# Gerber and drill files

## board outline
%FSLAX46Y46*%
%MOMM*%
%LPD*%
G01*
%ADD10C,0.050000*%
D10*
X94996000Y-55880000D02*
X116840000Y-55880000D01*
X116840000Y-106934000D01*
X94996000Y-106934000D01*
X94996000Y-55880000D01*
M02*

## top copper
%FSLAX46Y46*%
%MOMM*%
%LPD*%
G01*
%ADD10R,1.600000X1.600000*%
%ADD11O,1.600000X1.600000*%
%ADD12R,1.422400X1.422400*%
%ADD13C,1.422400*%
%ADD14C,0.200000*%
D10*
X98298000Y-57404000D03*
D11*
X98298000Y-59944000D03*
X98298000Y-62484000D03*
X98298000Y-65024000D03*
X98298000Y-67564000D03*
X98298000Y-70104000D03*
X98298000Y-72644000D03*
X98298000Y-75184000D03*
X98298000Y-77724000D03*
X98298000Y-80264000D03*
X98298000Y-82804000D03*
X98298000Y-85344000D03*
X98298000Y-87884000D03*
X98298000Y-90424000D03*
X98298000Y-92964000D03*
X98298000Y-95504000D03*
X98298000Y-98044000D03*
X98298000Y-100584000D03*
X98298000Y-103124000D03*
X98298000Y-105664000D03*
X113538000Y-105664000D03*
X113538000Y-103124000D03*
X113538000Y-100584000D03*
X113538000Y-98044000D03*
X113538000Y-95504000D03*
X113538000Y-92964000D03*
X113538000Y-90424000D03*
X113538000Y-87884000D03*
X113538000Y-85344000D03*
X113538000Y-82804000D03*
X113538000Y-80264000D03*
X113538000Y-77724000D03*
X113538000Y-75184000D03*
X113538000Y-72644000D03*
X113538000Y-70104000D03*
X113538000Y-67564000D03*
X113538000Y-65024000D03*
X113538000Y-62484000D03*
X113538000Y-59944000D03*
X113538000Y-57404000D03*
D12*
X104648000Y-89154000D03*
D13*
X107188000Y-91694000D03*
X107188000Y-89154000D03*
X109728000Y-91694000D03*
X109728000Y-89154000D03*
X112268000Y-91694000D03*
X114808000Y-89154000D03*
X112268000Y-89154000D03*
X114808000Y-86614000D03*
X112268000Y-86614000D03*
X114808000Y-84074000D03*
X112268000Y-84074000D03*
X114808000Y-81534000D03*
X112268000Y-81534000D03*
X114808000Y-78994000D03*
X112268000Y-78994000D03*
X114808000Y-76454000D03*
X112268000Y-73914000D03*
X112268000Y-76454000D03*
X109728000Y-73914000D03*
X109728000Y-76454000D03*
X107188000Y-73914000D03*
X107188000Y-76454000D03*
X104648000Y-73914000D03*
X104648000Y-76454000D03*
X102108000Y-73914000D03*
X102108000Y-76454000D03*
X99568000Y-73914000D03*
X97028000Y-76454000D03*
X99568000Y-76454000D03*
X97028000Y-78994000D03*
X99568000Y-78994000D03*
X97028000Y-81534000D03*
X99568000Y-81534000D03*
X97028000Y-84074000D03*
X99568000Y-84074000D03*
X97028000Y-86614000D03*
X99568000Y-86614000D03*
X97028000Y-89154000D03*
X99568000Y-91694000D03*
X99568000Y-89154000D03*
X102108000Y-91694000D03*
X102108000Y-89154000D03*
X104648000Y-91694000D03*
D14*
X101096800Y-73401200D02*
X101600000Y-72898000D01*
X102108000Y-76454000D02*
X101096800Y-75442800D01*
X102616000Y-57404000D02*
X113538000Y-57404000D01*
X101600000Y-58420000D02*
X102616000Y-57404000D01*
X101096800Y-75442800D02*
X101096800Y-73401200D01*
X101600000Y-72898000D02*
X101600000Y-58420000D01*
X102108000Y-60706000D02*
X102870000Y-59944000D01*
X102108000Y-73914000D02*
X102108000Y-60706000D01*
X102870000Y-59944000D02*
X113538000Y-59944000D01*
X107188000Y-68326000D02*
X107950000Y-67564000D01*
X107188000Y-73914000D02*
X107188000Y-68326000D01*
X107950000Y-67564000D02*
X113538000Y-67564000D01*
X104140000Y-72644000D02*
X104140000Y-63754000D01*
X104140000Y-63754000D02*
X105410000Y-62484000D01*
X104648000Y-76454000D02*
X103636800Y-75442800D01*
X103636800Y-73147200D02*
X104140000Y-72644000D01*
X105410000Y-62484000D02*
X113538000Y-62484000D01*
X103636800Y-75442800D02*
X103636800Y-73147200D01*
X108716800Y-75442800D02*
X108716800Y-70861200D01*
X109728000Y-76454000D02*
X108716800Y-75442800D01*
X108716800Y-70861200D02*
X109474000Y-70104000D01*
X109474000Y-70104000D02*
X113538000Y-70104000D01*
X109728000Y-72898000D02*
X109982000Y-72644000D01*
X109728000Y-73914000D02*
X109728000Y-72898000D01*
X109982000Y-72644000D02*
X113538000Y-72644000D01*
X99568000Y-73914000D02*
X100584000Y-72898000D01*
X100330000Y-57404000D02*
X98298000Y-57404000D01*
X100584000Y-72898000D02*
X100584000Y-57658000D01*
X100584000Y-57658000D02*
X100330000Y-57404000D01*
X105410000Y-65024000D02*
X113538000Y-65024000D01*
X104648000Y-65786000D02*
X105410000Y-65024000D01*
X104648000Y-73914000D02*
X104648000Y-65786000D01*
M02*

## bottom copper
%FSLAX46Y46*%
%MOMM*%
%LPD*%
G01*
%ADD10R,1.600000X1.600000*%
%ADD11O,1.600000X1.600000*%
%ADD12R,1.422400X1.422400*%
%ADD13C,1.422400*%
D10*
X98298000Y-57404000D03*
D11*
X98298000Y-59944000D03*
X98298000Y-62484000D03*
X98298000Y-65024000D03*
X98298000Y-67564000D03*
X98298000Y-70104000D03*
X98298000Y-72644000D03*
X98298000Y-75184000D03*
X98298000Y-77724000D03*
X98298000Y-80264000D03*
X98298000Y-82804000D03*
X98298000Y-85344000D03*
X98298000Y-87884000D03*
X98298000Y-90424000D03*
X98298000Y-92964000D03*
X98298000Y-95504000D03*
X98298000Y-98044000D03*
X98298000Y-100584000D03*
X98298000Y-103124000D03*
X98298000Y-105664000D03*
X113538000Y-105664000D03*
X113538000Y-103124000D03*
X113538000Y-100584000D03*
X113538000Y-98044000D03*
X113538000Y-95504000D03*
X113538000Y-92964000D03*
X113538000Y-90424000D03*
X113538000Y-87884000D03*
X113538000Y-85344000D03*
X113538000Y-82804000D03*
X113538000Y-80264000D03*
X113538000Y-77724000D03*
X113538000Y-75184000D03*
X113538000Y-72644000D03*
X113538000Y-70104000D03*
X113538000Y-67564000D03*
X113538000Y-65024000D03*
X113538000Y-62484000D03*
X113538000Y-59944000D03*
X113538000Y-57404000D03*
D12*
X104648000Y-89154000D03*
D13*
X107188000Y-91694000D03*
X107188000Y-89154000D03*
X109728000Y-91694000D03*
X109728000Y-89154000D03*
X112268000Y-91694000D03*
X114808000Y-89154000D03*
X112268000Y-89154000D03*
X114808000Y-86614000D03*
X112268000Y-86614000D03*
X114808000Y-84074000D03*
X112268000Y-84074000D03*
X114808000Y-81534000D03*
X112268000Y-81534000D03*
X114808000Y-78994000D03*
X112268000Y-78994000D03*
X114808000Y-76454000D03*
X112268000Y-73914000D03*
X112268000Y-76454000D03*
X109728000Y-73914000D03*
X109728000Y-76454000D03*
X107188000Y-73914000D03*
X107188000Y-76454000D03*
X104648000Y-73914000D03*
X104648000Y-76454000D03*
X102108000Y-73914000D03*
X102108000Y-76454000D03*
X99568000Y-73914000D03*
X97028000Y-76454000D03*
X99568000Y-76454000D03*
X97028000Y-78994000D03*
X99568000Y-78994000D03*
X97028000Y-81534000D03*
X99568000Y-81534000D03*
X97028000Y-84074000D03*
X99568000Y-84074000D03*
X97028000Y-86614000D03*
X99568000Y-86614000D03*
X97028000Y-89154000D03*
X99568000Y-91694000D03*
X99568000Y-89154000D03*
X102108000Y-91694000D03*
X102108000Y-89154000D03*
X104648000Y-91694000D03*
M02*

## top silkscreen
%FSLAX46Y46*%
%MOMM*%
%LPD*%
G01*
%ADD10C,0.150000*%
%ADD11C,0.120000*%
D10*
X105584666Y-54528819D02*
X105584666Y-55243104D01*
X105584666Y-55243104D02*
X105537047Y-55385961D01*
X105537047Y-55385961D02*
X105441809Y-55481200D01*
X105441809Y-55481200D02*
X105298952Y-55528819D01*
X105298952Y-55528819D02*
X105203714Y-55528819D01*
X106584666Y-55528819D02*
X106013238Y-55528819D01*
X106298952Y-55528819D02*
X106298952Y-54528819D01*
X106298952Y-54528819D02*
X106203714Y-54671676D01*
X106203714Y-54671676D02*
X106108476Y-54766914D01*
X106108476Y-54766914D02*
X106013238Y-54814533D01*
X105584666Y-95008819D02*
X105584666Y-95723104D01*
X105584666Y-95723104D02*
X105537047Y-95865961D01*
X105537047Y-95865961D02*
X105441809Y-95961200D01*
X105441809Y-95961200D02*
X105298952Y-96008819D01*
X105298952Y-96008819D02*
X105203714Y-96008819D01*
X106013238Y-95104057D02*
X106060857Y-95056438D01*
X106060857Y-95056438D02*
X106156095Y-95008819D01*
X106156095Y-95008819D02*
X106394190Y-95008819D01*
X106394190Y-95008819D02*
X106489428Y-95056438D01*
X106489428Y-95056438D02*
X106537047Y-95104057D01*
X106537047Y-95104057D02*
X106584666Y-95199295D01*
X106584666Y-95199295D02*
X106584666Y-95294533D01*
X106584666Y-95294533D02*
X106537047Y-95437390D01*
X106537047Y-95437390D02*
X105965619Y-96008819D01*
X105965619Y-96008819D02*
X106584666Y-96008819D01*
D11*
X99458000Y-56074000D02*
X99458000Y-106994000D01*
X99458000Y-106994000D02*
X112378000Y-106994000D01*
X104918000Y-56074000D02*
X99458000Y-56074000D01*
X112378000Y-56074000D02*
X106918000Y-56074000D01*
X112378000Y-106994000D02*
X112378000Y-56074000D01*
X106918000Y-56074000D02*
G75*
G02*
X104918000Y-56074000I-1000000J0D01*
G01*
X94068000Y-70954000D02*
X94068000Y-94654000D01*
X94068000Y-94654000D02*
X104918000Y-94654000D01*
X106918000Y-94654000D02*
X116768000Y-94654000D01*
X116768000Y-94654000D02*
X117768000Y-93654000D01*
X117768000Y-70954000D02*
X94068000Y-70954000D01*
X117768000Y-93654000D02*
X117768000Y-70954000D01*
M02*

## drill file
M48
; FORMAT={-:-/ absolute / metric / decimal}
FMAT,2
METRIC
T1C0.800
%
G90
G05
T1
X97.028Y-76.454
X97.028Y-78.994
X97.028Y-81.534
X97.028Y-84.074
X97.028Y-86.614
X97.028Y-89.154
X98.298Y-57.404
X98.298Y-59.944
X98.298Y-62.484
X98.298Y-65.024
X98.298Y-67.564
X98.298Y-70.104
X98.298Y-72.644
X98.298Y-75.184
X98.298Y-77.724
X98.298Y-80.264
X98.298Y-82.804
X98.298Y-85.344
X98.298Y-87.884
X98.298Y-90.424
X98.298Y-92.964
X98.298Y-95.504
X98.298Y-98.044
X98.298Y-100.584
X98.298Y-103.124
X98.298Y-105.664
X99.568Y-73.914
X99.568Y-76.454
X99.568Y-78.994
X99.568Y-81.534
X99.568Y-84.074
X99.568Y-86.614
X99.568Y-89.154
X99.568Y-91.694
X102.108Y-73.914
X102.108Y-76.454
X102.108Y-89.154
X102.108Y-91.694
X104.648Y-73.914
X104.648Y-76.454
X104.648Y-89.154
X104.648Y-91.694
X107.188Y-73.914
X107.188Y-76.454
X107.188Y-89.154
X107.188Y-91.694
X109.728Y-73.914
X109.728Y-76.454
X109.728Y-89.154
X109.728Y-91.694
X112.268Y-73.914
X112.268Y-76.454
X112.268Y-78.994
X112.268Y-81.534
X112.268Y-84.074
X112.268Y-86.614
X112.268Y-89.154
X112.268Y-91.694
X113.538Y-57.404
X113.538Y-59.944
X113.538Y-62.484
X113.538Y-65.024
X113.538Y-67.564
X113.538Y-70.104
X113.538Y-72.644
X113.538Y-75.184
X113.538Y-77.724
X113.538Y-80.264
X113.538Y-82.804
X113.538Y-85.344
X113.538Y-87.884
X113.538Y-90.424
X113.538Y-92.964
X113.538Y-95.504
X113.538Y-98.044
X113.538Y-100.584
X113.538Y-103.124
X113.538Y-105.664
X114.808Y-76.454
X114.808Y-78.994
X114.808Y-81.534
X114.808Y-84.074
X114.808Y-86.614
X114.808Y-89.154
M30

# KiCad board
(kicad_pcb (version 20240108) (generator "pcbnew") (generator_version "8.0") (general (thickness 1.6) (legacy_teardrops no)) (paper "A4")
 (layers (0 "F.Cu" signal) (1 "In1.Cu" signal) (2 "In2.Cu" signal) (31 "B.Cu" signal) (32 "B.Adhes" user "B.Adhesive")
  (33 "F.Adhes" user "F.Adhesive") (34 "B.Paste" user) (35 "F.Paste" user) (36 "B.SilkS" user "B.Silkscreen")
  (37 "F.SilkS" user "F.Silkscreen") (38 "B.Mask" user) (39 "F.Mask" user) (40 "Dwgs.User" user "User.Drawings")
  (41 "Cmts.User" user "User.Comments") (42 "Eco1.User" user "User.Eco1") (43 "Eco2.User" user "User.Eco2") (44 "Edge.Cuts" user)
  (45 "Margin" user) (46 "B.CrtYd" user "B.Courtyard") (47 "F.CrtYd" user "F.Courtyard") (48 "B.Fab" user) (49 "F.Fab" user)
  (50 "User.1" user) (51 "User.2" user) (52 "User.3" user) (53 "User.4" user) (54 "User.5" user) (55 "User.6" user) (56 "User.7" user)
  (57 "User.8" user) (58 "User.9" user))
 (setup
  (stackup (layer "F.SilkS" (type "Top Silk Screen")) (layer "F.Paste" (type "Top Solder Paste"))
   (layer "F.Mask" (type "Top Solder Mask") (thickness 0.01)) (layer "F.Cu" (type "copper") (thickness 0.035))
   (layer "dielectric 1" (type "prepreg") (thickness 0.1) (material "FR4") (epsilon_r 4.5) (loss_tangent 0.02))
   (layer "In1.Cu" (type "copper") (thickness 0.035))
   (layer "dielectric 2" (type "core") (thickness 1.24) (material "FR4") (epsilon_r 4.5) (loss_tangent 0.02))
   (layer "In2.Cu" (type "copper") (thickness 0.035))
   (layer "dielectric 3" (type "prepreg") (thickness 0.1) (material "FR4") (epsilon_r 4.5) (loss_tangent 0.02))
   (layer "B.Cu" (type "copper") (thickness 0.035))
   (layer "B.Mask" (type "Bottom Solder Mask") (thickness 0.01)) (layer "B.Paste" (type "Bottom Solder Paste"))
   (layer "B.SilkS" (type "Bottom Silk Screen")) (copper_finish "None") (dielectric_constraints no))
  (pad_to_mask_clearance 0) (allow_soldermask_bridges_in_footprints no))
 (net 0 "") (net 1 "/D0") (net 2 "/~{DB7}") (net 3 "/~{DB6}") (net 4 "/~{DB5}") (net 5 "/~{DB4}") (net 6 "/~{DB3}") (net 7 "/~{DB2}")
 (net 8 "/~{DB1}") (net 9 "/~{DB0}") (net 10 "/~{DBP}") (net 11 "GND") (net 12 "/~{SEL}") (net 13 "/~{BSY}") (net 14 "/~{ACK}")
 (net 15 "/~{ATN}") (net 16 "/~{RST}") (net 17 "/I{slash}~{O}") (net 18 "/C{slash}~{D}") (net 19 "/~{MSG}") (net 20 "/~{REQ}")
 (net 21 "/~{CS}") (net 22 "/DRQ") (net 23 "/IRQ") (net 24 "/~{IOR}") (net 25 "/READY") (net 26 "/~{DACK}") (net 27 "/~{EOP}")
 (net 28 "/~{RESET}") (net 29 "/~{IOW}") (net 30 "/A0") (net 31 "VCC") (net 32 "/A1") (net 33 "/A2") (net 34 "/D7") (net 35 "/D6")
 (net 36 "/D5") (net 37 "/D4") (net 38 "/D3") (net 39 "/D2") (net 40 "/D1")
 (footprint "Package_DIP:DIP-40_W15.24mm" (layer "F.Cu") (at 98.298 57.404)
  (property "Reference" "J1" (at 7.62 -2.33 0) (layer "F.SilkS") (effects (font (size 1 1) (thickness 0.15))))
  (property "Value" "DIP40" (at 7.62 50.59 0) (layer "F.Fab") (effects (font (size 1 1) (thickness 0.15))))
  (fp_line (start 1.16 -1.33) (end 1.16 49.59) (stroke (width 0.12) (type solid)) (layer "F.SilkS"))
  (fp_line (start 1.16 49.59) (end 14.08 49.59) (stroke (width 0.12) (type solid)) (layer "F.SilkS"))
  (fp_line (start 6.62 -1.33) (end 1.16 -1.33) (stroke (width 0.12) (type solid)) (layer "F.SilkS"))
  (fp_line (start 14.08 -1.33) (end 8.62 -1.33) (stroke (width 0.12) (type solid)) (layer "F.SilkS"))
  (fp_line (start 14.08 49.59) (end 14.08 -1.33) (stroke (width 0.12) (type solid)) (layer "F.SilkS"))
  (fp_arc (start 8.62 -1.33) (mid 7.62 -0.33) (end 6.62 -1.33) (stroke (width 0.12) (type solid)) (layer "F.SilkS"))
  (pad "1" thru_hole rect (at 0 0) (size 1.6 1.6) (drill 0.8) (layers "*.Cu" "*.Mask") (remove_unused_layers no) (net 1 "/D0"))
  (pad "2" thru_hole oval (at 0 2.54) (size 1.6 1.6) (drill 0.8) (layers "*.Cu" "*.Mask") (remove_unused_layers no) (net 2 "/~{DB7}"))
  (pad "3" thru_hole oval (at 0 5.08) (size 1.6 1.6) (drill 0.8) (layers "*.Cu" "*.Mask") (remove_unused_layers no) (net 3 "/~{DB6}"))
  (pad "4" thru_hole oval (at 0 7.62) (size 1.6 1.6) (drill 0.8) (layers "*.Cu" "*.Mask") (remove_unused_layers no) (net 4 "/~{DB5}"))
  (pad "5" thru_hole oval (at 0 10.16) (size 1.6 1.6) (drill 0.8) (layers "*.Cu" "*.Mask") (remove_unused_layers no) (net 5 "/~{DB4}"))
  (pad "6" thru_hole oval (at 0 12.7) (size 1.6 1.6) (drill 0.8) (layers "*.Cu" "*.Mask") (remove_unused_layers no) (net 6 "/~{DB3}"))
  (pad "7" thru_hole oval (at 0 15.24) (size 1.6 1.6) (drill 0.8) (layers "*.Cu" "*.Mask") (remove_unused_layers no) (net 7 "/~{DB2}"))
  (pad "8" thru_hole oval (at 0 17.78) (size 1.6 1.6) (drill 0.8) (layers "*.Cu" "*.Mask") (remove_unused_layers no) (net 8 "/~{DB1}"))
  (pad "9" thru_hole oval (at 0 20.32) (size 1.6 1.6) (drill 0.8) (layers "*.Cu" "*.Mask") (remove_unused_layers no) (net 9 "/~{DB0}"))
  (pad "10" thru_hole oval (at 0 22.86) (size 1.6 1.6) (drill 0.8) (layers "*.Cu" "*.Mask") (remove_unused_layers no) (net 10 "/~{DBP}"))
  (pad "11" thru_hole oval (at 0 25.4) (size 1.6 1.6) (drill 0.8) (layers "*.Cu" "*.Mask") (remove_unused_layers no) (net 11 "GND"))
  (pad "12" thru_hole oval (at 0 27.94) (size 1.6 1.6) (drill 0.8) (layers "*.Cu" "*.Mask") (remove_unused_layers no) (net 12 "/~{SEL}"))
  (pad "13" thru_hole oval (at 0 30.48) (size 1.6 1.6) (drill 0.8) (layers "*.Cu" "*.Mask") (remove_unused_layers no) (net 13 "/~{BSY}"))
  (pad "14" thru_hole oval (at 0 33.02) (size 1.6 1.6) (drill 0.8) (layers "*.Cu" "*.Mask") (remove_unused_layers no) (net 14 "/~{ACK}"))
  (pad "15" thru_hole oval (at 0 35.56) (size 1.6 1.6) (drill 0.8) (layers "*.Cu" "*.Mask") (remove_unused_layers no) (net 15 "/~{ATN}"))
  (pad "16" thru_hole oval (at 0 38.1) (size 1.6 1.6) (drill 0.8) (layers "*.Cu" "*.Mask") (remove_unused_layers no) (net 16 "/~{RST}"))
  (pad "17" thru_hole oval (at 0 40.64) (size 1.6 1.6) (drill 0.8) (layers "*.Cu" "*.Mask") (remove_unused_layers no)
   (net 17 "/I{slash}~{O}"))
  (pad "18" thru_hole oval (at 0 43.18) (size 1.6 1.6) (drill 0.8) (layers "*.Cu" "*.Mask") (remove_unused_layers no)
   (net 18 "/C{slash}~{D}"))
  (pad "19" thru_hole oval (at 0 45.72) (size 1.6 1.6) (drill 0.8) (layers "*.Cu" "*.Mask") (remove_unused_layers no) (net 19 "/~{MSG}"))
  (pad "20" thru_hole oval (at 0 48.26) (size 1.6 1.6) (drill 0.8) (layers "*.Cu" "*.Mask") (remove_unused_layers no) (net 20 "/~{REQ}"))
  (pad "21" thru_hole oval (at 15.24 48.26) (size 1.6 1.6) (drill 0.8) (layers "*.Cu" "*.Mask") (remove_unused_layers no) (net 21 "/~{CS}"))
  (pad "22" thru_hole oval (at 15.24 45.72) (size 1.6 1.6) (drill 0.8) (layers "*.Cu" "*.Mask") (remove_unused_layers no) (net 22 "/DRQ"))
  (pad "23" thru_hole oval (at 15.24 43.18) (size 1.6 1.6) (drill 0.8) (layers "*.Cu" "*.Mask") (remove_unused_layers no) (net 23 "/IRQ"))
  (pad "24" thru_hole oval (at 15.24 40.64) (size 1.6 1.6) (drill 0.8) (layers "*.Cu" "*.Mask") (remove_unused_layers no) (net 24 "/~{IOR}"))
  (pad "25" thru_hole oval (at 15.24 38.1) (size 1.6 1.6) (drill 0.8) (layers "*.Cu" "*.Mask") (remove_unused_layers no) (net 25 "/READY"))
  (pad "26" thru_hole oval (at 15.24 35.56) (size 1.6 1.6) (drill 0.8) (layers "*.Cu" "*.Mask") (remove_unused_layers no)
   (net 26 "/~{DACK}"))
  (pad "27" thru_hole oval (at 15.24 33.02) (size 1.6 1.6) (drill 0.8) (layers "*.Cu" "*.Mask") (remove_unused_layers no) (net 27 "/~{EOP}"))
  (pad "28" thru_hole oval (at 15.24 30.48) (size 1.6 1.6) (drill 0.8) (layers "*.Cu" "*.Mask") (remove_unused_layers no)
   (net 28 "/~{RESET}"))
  (pad "29" thru_hole oval (at 15.24 27.94) (size 1.6 1.6) (drill 0.8) (layers "*.Cu" "*.Mask") (remove_unused_layers no) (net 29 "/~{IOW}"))
  (pad "30" thru_hole oval (at 15.24 25.4) (size 1.6 1.6) (drill 0.8) (layers "*.Cu" "*.Mask") (remove_unused_layers no) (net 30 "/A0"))
  (pad "31" thru_hole oval (at 15.24 22.86) (size 1.6 1.6) (drill 0.8) (layers "*.Cu" "*.Mask") (remove_unused_layers no) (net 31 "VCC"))
  (pad "32" thru_hole oval (at 15.24 20.32) (size 1.6 1.6) (drill 0.8) (layers "*.Cu" "*.Mask") (remove_unused_layers no) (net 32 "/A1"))
  (pad "33" thru_hole oval (at 15.24 17.78) (size 1.6 1.6) (drill 0.8) (layers "*.Cu" "*.Mask") (remove_unused_layers no) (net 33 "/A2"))
  (pad "34" thru_hole oval (at 15.24 15.24) (size 1.6 1.6) (drill 0.8) (layers "*.Cu" "*.Mask") (remove_unused_layers no) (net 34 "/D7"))
  (pad "35" thru_hole oval (at 15.24 12.7) (size 1.6 1.6) (drill 0.8) (layers "*.Cu" "*.Mask") (remove_unused_layers no) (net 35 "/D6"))
  (pad "36" thru_hole oval (at 15.24 10.16) (size 1.6 1.6) (drill 0.8) (layers "*.Cu" "*.Mask") (remove_unused_layers no) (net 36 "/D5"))
  (pad "37" thru_hole oval (at 15.24 7.62) (size 1.6 1.6) (drill 0.8) (layers "*.Cu" "*.Mask") (remove_unused_layers no) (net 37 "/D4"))
  (pad "38" thru_hole oval (at 15.24 5.08) (size 1.6 1.6) (drill 0.8) (layers "*.Cu" "*.Mask") (remove_unused_layers no) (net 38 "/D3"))
  (pad "39" thru_hole oval (at 15.24 2.54) (size 1.6 1.6) (drill 0.8) (layers "*.Cu" "*.Mask") (remove_unused_layers no) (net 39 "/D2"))
  (pad "40" thru_hole oval (at 15.24 0) (size 1.6 1.6) (drill 0.8) (layers "*.Cu" "*.Mask") (remove_unused_layers no) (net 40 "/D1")))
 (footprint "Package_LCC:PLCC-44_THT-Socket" (layer "F.Cu") (at 104.648 89.154 180)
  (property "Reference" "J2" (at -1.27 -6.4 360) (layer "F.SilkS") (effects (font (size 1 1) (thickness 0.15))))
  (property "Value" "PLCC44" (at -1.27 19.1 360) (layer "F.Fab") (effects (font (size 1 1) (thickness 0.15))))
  (fp_line (start 10.58 18.2) (end 10.58 -5.5) (stroke (width 0.12) (type solid)) (layer "F.SilkS"))
  (fp_line (start 10.58 -5.5) (end -0.27 -5.5) (stroke (width 0.12) (type solid)) (layer "F.SilkS"))
  (fp_line (start -2.27 -5.5) (end -12.12 -5.5) (stroke (width 0.12) (type solid)) (layer "F.SilkS"))
  (fp_line (start -12.12 -5.5) (end -13.12 -4.5) (stroke (width 0.12) (type solid)) (layer "F.SilkS"))
  (fp_line (start -13.12 18.2) (end 10.58 18.2) (stroke (width 0.12) (type solid)) (layer "F.SilkS"))
  (fp_line (start -13.12 -4.5) (end -13.12 18.2) (stroke (width 0.12) (type solid)) (layer "F.SilkS"))
  (pad "1" thru_hole rect (at 0 0 180) (size 1.4224 1.4224) (drill 0.8) (layers "*.Cu" "*.Mask") (remove_unused_layers no) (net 2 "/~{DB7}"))
  (pad "2" thru_hole circle (at -2.54 -2.54 180) (size 1.4224 1.4224) (drill 0.8) (layers "*.Cu" "*.Mask") (remove_unused_layers no)
   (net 16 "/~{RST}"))
  (pad "3" thru_hole circle (at -2.54 0 180) (size 1.4224 1.4224) (drill 0.8) (layers "*.Cu" "*.Mask") (remove_unused_layers no)
   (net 11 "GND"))
  (pad "4" thru_hole circle (at -5.08 -2.54 180) (size 1.4224 1.4224) (drill 0.8) (layers "*.Cu" "*.Mask") (remove_unused_layers no)
   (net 13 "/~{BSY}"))
  (pad "5" thru_hole circle (at -5.08 0 180) (size 1.4224 1.4224) (drill 0.8) (layers "*.Cu" "*.Mask") (remove_unused_layers no)
   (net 12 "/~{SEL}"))
  (pad "6" thru_hole circle (at -7.62 -2.54 180) (size 1.4224 1.4224) (drill 0.8) (layers "*.Cu" "*.Mask") (remove_unused_layers no)
   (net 15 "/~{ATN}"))
  (pad "7" thru_hole circle (at -10.16 0 180) (size 1.4224 1.4224) (drill 0.8) (layers "*.Cu" "*.Mask") (remove_unused_layers no)
   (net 28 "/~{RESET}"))
  (pad "8" thru_hole circle (at -7.62 0 180) (size 1.4224 1.4224) (drill 0.8) (layers "*.Cu" "*.Mask") (remove_unused_layers no)
   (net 23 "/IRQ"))
  (pad "9" thru_hole circle (at -10.16 2.54 180) (size 1.4224 1.4224) (drill 0.8) (layers "*.Cu" "*.Mask") (remove_unused_layers no)
   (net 22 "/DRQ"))
  (pad "10" thru_hole circle (at -7.62 2.54 180) (size 1.4224 1.4224) (drill 0.8) (layers "*.Cu" "*.Mask") (remove_unused_layers no)
   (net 27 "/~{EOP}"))
  (pad "11" thru_hole circle (at -10.16 5.08 180) (size 1.4224 1.4224) (drill 0.8) (layers "*.Cu" "*.Mask") (remove_unused_layers no)
   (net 26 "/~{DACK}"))
  (pad "12" thru_hole circle (at -7.62 5.08 180) (size 1.4224 1.4224) (drill 0.8) (layers "*.Cu" "*.Mask") (remove_unused_layers no)
   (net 11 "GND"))
  (pad "13" thru_hole circle (at -10.16 7.62 180) (size 1.4224 1.4224) (drill 0.8) (layers "*.Cu" "*.Mask") (remove_unused_layers no)
   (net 25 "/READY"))
  (pad "14" thru_hole circle (at -7.62 7.62 180) (size 1.4224 1.4224) (drill 0.8) (layers "*.Cu" "*.Mask") (remove_unused_layers no)
   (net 30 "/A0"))
  (pad "15" thru_hole circle (at -10.16 10.16 180) (size 1.4224 1.4224) (drill 0.8) (layers "*.Cu" "*.Mask") (remove_unused_layers no)
   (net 32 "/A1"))
  (pad "16" thru_hole circle (at -7.62 10.16 180) (size 1.4224 1.4224) (drill 0.8) (layers "*.Cu" "*.Mask") (remove_unused_layers no)
   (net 33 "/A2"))
  (pad "17" thru_hole circle (at -10.16 12.7 180) (size 1.4224 1.4224) (drill 0.8) (layers "*.Cu" "*.Mask") (remove_unused_layers no)
   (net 21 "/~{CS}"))
  (pad "18" thru_hole circle (at -7.62 15.24 180) (size 1.4224 1.4224) (drill 0.8) (layers "*.Cu" "*.Mask") (remove_unused_layers no)
   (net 29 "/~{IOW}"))
  (pad "19" thru_hole circle (at -7.62 12.7 180) (size 1.4224 1.4224) (drill 0.8) (layers "*.Cu" "*.Mask") (remove_unused_layers no)
   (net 24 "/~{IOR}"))
  (pad "20" thru_hole circle (at -5.08 15.24 180) (size 1.4224 1.4224) (drill 0.8) (layers "*.Cu" "*.Mask") (remove_unused_layers no)
   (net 34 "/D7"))
  (pad "21" thru_hole circle (at -5.08 12.7 180) (size 1.4224 1.4224) (drill 0.8) (layers "*.Cu" "*.Mask") (remove_unused_layers no)
   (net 35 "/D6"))
  (pad "22" thru_hole circle (at -2.54 15.24 180) (size 1.4224 1.4224) (drill 0.8) (layers "*.Cu" "*.Mask") (remove_unused_layers no)
   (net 36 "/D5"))
  (pad "23" thru_hole circle (at -2.54 12.7 180) (size 1.4224 1.4224) (drill 0.8) (layers "*.Cu" "*.Mask") (remove_unused_layers no)
   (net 31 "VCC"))
  (pad "24" thru_hole circle (at 0 15.24 180) (size 1.4224 1.4224) (drill 0.8) (layers "*.Cu" "*.Mask") (remove_unused_layers no)
   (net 37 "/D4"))
  (pad "25" thru_hole circle (at 0 12.7 180) (size 1.4224 1.4224) (drill 0.8) (layers "*.Cu" "*.Mask") (remove_unused_layers no)
   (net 38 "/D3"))
  (pad "26" thru_hole circle (at 2.54 15.24 180) (size 1.4224 1.4224) (drill 0.8) (layers "*.Cu" "*.Mask") (remove_unused_layers no)
   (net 39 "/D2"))
  (pad "27" thru_hole circle (at 2.54 12.7 180) (size 1.4224 1.4224) (drill 0.8) (layers "*.Cu" "*.Mask") (remove_unused_layers no)
   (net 40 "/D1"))
  (pad "28" thru_hole circle (at 5.08 15.24 180) (size 1.4224 1.4224) (drill 0.8) (layers "*.Cu" "*.Mask") (remove_unused_layers no)
   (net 1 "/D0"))
  (pad "29" thru_hole circle (at 7.62 12.7 180) (size 1.4224 1.4224) (drill 0.8) (layers "*.Cu" "*.Mask") (remove_unused_layers no)
   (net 19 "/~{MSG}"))
  (pad "30" thru_hole circle (at 5.08 12.7 180) (size 1.4224 1.4224) (drill 0.8) (layers "*.Cu" "*.Mask") (remove_unused_layers no)
   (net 18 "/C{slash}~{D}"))
  (pad "31" thru_hole circle (at 7.62 10.16 180) (size 1.4224 1.4224) (drill 0.8) (layers "*.Cu" "*.Mask") (remove_unused_layers no)
   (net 11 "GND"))
  (pad "32" thru_hole circle (at 5.08 10.16 180) (size 1.4224 1.4224) (drill 0.8) (layers "*.Cu" "*.Mask") (remove_unused_layers no)
   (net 17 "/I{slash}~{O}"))
  (pad "33" thru_hole circle (at 7.62 7.62 180) (size 1.4224 1.4224) (drill 0.8) (layers "*.Cu" "*.Mask") (remove_unused_layers no)
   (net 14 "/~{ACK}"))
  (pad "34" thru_hole circle (at 5.08 7.62 180) (size 1.4224 1.4224) (drill 0.8) (layers "*.Cu" "*.Mask") (remove_unused_layers no)
   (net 20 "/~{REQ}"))
  (pad "35" thru_hole circle (at 7.62 5.08 180) (size 1.4224 1.4224) (drill 0.8) (layers "*.Cu" "*.Mask") (remove_unused_layers no)
   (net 10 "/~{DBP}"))
  (pad "36" thru_hole circle (at 5.08 5.08 180) (size 1.4224 1.4224) (drill 0.8) (layers "*.Cu" "*.Mask") (remove_unused_layers no)
   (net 11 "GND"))
  (pad "37" thru_hole circle (at 7.62 2.54 180) (size 1.4224 1.4224) (drill 0.8) (layers "*.Cu" "*.Mask") (remove_unused_layers no)
   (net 9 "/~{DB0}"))
  (pad "38" thru_hole circle (at 5.08 2.54 180) (size 1.4224 1.4224) (drill 0.8) (layers "*.Cu" "*.Mask") (remove_unused_layers no)
   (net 8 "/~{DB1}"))
  (pad "39" thru_hole circle (at 7.62 0 180) (size 1.4224 1.4224) (drill 0.8) (layers "*.Cu" "*.Mask") (remove_unused_layers no)
   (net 7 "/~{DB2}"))
  (pad "40" thru_hole circle (at 5.08 -2.54 180) (size 1.4224 1.4224) (drill 0.8) (layers "*.Cu" "*.Mask") (remove_unused_layers no)
   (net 6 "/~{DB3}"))
  (pad "41" thru_hole circle (at 5.08 0 180) (size 1.4224 1.4224) (drill 0.8) (layers "*.Cu" "*.Mask") (remove_unused_layers no)
   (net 5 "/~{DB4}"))
  (pad "42" thru_hole circle (at 2.54 -2.54 180) (size 1.4224 1.4224) (drill 0.8) (layers "*.Cu" "*.Mask") (remove_unused_layers no)
   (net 11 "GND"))
  (pad "43" thru_hole circle (at 2.54 0 180) (size 1.4224 1.4224) (drill 0.8) (layers "*.Cu" "*.Mask") (remove_unused_layers no)
   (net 4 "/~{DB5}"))
  (pad "44" thru_hole circle (at 0 -2.54 180) (size 1.4224 1.4224) (drill 0.8) (layers "*.Cu" "*.Mask") (remove_unused_layers no)
   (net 3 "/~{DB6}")))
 (gr_rect (start 94.996 55.88) (end 116.84 106.934) (stroke (width 0.05) (type default)) (fill none) (layer "Edge.Cuts"))
 (segment (start 101.0968 73.4012) (end 101.6 72.898) (width 0.2) (layer "F.Cu") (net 40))
 (segment (start 102.108 76.454) (end 101.0968 75.4428) (width 0.2) (layer "F.Cu") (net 40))
 (segment (start 102.616 57.404) (end 113.538 57.404) (width 0.2) (layer "F.Cu") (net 40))
 (segment (start 101.6 58.42) (end 102.616 57.404) (width 0.2) (layer "F.Cu") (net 40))
 (segment (start 101.0968 75.4428) (end 101.0968 73.4012) (width 0.2) (layer "F.Cu") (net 40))
 (segment (start 101.6 72.898) (end 101.6 58.42) (width 0.2) (layer "F.Cu") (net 40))
 (segment (start 102.108 60.706) (end 102.87 59.944) (width 0.2) (layer "F.Cu") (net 39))
 (segment (start 102.108 73.914) (end 102.108 60.706) (width 0.2) (layer "F.Cu") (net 39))
 (segment (start 102.87 59.944) (end 113.538 59.944) (width 0.2) (layer "F.Cu") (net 39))
 (segment (start 107.188 68.326) (end 107.95 67.564) (width 0.2) (layer "F.Cu") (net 36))
 (segment (start 107.188 73.914) (end 107.188 68.326) (width 0.2) (layer "F.Cu") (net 36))
 (segment (start 107.95 67.564) (end 113.538 67.564) (width 0.2) (layer "F.Cu") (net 36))
 (segment (start 104.14 72.644) (end 104.14 63.754) (width 0.2) (layer "F.Cu") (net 38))
 (segment (start 104.14 63.754) (end 105.41 62.484) (width 0.2) (layer "F.Cu") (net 38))
 (segment (start 104.648 76.454) (end 103.6368 75.4428) (width 0.2) (layer "F.Cu") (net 38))
 (segment (start 103.6368 73.1472) (end 104.14 72.644) (width 0.2) (layer "F.Cu") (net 38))
 (segment (start 105.41 62.484) (end 113.538 62.484) (width 0.2) (layer "F.Cu") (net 38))
 (segment (start 103.6368 75.4428) (end 103.6368 73.1472) (width 0.2) (layer "F.Cu") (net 38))
 (segment (start 108.7168 75.4428) (end 108.7168 70.8612) (width 0.2) (layer "F.Cu") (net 35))
 (segment (start 109.728 76.454) (end 108.7168 75.4428) (width 0.2) (layer "F.Cu") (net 35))
 (segment (start 108.7168 70.8612) (end 109.474 70.104) (width 0.2) (layer "F.Cu") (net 35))
 (segment (start 109.474 70.104) (end 113.538 70.104) (width 0.2) (layer "F.Cu") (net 35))
 (segment (start 109.728 72.898) (end 109.982 72.644) (width 0.2) (layer "F.Cu") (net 34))
 (segment (start 109.728 73.914) (end 109.728 72.898) (width 0.2) (layer "F.Cu") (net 34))
 (segment (start 109.982 72.644) (end 113.538 72.644) (width 0.2) (layer "F.Cu") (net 34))
 (segment (start 99.568 73.914) (end 100.584 72.898) (width 0.2) (layer "F.Cu") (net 1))
 (segment (start 100.33 57.404) (end 98.298 57.404) (width 0.2) (layer "F.Cu") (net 1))
 (segment (start 100.584 72.898) (end 100.584 57.658) (width 0.2) (layer "F.Cu") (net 1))
 (segment (start 100.584 57.658) (end 100.33 57.404) (width 0.2) (layer "F.Cu") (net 1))
 (segment (start 105.41 65.024) (end 113.538 65.024) (width 0.2) (layer "F.Cu") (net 37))
 (segment (start 104.648 65.786) (end 105.41 65.024) (width 0.2) (layer "F.Cu") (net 37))
 (segment (start 104.648 73.914) (end 104.648 65.786) (width 0.2) (layer "F.Cu") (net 37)))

